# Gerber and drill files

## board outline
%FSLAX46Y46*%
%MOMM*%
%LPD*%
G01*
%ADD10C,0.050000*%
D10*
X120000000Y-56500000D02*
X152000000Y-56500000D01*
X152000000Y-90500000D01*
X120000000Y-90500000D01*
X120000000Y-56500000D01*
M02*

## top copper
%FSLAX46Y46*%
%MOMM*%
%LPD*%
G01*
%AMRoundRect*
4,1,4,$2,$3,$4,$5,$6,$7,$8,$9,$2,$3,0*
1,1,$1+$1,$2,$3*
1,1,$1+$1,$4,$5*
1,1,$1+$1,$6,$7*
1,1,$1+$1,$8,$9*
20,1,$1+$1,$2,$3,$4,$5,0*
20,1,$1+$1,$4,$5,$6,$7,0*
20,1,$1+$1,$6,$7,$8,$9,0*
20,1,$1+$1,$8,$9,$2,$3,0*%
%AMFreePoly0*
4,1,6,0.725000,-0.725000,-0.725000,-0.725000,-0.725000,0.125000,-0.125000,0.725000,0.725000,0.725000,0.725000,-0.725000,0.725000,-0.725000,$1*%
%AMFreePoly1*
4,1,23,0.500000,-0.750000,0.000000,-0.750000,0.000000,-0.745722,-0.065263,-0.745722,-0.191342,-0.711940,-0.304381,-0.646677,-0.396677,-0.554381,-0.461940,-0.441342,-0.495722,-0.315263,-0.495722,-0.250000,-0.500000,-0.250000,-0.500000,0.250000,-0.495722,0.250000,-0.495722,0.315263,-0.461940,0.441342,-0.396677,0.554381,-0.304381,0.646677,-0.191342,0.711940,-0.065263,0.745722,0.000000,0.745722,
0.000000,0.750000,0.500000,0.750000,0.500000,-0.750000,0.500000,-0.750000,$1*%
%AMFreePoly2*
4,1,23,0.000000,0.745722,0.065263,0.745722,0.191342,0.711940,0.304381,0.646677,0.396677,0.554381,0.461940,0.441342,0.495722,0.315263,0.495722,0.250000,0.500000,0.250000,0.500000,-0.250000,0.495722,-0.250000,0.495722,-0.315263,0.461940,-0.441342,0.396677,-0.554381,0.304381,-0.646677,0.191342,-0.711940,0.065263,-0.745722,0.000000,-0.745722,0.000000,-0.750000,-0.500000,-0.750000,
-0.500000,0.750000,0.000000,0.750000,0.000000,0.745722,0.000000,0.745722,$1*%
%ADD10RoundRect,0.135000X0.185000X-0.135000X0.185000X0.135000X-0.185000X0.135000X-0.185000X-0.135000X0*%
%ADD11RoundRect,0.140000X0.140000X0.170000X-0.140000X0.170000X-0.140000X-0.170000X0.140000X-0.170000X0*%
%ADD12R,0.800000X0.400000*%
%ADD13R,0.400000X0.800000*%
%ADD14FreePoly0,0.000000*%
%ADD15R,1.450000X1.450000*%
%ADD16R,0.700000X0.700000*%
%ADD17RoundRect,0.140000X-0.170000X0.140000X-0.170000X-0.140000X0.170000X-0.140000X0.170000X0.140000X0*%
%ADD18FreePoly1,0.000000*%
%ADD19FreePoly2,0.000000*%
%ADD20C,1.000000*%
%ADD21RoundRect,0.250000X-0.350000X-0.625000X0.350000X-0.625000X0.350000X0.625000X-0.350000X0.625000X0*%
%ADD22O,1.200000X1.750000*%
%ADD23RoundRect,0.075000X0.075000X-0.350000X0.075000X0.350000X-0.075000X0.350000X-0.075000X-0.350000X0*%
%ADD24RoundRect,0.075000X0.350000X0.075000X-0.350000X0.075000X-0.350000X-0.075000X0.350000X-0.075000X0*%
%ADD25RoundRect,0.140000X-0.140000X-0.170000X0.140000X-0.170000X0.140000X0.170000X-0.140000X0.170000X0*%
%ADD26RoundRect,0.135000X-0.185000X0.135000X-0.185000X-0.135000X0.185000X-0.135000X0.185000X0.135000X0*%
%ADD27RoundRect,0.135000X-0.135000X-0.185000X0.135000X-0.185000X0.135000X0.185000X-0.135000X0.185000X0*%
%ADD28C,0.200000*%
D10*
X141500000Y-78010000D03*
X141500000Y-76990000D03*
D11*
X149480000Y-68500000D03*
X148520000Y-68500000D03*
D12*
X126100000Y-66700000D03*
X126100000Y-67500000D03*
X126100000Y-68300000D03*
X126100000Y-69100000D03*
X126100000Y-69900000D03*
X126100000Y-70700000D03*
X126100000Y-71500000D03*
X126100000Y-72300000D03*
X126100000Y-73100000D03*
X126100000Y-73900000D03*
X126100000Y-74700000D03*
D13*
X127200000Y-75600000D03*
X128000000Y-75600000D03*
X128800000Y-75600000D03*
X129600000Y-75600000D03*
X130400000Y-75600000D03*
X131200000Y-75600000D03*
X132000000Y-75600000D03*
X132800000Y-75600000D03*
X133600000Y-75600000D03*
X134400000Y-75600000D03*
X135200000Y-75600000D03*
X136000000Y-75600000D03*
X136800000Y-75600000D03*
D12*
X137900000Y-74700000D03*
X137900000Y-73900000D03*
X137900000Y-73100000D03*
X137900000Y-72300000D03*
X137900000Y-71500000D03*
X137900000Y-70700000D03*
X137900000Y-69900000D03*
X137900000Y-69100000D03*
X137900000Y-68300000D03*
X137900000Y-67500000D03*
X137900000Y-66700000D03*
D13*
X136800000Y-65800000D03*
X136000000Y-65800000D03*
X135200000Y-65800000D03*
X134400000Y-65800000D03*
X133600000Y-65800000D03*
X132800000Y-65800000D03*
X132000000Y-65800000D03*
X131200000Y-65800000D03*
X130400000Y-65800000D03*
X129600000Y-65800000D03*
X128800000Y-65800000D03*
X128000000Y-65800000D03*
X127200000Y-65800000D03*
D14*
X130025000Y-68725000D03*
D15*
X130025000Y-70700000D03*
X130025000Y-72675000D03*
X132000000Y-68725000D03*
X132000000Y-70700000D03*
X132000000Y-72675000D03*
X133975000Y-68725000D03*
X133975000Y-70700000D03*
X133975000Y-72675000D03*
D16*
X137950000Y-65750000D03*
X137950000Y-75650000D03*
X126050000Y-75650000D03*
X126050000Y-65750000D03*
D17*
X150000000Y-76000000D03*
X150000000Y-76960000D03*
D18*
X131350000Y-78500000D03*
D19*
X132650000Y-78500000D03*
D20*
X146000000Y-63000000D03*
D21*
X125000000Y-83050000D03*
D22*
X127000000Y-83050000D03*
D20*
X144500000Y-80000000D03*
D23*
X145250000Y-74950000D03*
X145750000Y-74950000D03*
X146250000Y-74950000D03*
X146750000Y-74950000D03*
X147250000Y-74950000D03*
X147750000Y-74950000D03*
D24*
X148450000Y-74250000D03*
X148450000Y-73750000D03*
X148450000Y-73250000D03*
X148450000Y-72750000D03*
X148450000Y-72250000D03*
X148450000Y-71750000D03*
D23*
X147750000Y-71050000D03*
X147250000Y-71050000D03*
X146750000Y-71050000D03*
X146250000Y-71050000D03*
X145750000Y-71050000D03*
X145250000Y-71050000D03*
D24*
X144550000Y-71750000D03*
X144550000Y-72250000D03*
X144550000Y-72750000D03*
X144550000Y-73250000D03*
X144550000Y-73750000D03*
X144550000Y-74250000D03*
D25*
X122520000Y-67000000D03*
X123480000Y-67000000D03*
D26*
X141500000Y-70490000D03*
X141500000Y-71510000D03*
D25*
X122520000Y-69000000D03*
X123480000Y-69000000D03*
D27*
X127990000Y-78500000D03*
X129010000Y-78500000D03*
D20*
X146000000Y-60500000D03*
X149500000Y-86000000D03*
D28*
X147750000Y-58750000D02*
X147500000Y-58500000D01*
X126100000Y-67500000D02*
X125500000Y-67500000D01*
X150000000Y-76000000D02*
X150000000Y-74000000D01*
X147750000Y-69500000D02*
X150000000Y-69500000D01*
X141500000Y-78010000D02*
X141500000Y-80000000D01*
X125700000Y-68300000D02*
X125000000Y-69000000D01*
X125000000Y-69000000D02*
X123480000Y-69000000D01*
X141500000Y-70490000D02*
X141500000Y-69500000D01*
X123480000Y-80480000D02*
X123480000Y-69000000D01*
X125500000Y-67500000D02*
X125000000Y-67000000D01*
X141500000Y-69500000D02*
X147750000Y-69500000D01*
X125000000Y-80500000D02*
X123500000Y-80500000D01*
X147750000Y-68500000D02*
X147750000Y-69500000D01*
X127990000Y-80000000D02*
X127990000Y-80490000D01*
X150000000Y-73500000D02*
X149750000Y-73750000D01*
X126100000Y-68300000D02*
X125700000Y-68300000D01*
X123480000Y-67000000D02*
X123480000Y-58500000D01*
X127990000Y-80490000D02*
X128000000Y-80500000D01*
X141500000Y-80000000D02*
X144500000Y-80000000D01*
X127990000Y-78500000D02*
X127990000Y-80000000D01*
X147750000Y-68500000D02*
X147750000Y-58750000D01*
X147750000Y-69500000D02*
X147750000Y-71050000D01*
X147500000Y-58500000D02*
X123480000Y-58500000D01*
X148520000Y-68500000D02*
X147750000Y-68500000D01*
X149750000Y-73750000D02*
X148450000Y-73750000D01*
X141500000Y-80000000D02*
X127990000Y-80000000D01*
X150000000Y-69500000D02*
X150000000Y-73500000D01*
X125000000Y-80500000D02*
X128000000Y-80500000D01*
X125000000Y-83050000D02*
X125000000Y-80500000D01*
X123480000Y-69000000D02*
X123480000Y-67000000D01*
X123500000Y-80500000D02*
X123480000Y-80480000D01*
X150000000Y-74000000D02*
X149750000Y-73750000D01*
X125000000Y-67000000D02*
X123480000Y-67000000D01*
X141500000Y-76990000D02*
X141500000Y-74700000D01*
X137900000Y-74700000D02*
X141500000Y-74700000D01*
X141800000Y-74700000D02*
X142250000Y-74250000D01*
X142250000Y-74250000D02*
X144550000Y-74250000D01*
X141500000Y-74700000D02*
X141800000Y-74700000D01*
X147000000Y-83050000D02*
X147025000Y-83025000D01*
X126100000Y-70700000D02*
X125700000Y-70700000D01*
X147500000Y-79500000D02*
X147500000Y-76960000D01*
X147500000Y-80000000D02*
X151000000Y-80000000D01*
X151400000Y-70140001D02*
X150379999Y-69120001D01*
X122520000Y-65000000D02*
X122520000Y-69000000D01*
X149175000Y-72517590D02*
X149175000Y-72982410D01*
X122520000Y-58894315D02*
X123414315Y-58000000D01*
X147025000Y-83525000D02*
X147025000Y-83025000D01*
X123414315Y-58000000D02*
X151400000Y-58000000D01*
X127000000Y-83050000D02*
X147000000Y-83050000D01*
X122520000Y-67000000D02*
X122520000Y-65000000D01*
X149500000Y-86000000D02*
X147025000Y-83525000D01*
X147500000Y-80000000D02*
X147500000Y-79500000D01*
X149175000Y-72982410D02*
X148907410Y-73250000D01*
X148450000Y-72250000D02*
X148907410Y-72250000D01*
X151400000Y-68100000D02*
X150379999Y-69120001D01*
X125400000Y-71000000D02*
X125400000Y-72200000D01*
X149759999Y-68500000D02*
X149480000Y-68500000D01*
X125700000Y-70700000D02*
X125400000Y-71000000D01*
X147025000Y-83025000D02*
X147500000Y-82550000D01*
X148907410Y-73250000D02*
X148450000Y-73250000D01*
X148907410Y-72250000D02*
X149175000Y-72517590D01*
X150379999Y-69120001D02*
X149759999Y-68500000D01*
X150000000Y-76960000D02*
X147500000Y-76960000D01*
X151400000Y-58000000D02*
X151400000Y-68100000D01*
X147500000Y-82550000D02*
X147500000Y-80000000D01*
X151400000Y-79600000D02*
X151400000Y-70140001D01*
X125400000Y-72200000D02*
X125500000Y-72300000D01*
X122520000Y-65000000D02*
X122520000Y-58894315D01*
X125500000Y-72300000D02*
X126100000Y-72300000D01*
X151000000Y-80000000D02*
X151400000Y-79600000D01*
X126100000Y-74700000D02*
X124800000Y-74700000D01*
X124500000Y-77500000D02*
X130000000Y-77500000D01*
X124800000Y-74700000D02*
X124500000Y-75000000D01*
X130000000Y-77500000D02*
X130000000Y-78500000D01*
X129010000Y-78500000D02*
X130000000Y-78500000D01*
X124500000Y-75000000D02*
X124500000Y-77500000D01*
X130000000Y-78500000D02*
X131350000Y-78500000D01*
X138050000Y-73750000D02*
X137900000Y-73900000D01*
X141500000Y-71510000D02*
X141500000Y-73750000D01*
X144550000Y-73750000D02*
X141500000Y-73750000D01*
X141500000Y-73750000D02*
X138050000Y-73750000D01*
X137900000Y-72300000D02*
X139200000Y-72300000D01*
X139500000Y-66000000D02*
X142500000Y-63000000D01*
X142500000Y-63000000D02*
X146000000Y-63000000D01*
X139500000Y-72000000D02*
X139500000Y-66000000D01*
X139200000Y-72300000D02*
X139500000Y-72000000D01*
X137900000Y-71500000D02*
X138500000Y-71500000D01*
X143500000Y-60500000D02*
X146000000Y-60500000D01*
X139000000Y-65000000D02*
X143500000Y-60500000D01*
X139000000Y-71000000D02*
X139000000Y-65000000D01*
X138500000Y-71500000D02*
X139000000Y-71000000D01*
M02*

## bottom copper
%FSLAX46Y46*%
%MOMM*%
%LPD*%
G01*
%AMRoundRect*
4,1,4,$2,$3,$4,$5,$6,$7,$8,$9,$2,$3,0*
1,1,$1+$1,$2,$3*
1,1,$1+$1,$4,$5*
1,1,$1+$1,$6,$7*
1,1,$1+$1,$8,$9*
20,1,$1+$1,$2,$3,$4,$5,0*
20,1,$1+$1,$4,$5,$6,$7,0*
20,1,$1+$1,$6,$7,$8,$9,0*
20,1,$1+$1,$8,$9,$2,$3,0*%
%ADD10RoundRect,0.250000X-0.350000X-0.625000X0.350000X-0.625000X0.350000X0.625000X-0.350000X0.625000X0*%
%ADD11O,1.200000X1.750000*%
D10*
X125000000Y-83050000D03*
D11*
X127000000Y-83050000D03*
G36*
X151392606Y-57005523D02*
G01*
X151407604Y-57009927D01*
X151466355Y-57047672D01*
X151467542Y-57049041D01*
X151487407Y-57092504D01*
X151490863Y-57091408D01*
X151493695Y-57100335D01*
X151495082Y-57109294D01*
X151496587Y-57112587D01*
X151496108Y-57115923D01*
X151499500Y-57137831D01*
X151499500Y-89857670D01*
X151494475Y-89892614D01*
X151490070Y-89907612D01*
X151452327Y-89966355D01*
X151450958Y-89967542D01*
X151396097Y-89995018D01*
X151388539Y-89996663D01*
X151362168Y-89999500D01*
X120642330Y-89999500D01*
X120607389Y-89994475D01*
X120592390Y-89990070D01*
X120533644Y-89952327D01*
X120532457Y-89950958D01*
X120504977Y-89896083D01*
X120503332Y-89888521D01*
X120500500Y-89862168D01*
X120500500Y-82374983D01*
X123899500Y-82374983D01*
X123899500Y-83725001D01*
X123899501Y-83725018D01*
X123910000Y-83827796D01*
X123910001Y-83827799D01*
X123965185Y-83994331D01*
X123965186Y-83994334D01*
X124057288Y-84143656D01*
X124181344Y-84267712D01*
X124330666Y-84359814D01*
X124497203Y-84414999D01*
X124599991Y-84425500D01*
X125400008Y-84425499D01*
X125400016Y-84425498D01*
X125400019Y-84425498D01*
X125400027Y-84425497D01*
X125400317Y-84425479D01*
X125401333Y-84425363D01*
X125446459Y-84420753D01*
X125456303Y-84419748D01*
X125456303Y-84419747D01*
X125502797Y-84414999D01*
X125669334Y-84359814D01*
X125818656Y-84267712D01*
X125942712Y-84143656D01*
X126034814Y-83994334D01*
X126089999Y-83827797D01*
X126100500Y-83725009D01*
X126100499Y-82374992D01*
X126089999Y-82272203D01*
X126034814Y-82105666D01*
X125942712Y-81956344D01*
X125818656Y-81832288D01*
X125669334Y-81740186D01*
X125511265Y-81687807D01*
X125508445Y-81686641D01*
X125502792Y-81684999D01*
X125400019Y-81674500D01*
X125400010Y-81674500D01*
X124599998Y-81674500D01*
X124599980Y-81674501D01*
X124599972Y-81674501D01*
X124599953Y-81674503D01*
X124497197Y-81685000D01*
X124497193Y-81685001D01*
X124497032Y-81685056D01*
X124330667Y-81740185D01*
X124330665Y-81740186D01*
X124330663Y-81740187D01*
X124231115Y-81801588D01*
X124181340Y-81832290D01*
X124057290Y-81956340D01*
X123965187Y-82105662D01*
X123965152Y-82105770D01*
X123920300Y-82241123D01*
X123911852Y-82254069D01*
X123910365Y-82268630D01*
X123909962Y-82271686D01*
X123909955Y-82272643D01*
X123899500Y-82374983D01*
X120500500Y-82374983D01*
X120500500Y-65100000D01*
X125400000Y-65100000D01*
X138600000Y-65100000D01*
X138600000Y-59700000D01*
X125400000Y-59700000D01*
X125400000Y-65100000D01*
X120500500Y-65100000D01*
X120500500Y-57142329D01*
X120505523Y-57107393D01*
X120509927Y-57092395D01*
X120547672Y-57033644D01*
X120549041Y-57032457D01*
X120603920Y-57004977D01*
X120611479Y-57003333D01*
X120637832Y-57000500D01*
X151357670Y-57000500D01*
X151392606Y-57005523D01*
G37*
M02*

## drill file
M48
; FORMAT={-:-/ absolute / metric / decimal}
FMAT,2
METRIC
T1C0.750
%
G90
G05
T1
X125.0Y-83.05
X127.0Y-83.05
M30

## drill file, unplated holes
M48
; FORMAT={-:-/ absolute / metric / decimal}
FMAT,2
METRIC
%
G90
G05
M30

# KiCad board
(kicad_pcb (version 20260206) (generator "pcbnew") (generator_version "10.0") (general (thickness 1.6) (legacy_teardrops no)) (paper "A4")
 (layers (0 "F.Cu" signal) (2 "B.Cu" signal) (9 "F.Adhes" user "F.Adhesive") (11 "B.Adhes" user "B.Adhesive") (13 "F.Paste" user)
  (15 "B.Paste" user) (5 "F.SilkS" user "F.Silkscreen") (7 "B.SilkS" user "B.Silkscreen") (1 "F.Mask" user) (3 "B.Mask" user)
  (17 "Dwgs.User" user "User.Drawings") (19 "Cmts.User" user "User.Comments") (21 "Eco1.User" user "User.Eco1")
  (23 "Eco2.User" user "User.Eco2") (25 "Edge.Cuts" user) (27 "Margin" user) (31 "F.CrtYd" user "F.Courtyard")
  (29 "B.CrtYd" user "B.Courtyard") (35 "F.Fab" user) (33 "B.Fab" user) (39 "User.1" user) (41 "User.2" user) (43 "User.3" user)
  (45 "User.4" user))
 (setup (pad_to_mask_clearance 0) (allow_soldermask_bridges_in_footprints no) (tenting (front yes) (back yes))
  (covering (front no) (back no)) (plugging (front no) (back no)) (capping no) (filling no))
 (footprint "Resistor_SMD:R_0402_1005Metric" (layer "F.Cu") (at 141.5 77.5 90)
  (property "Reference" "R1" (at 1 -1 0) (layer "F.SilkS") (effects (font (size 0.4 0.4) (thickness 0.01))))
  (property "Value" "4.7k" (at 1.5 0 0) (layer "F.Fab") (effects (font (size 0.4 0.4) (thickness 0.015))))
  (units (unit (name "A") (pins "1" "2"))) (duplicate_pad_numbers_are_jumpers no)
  (pad "1" smd roundrect (at -0.51 0 90) (size 0.54 0.64) (layers "F.Cu" "F.Mask" "F.Paste") (roundrect_rratio 0.25) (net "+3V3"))
  (pad "2" smd roundrect (at 0.51 0 90) (size 0.54 0.64) (layers "F.Cu" "F.Mask" "F.Paste") (roundrect_rratio 0.25) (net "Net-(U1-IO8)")))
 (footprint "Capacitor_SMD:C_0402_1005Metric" (layer "F.Cu") (at 149 68.5 180)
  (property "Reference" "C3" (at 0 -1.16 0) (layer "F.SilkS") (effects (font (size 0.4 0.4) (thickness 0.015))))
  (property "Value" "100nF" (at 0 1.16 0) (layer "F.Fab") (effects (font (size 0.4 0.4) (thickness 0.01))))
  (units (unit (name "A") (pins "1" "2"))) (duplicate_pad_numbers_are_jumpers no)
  (pad "1" smd roundrect (at -0.48 0 180) (size 0.56 0.62) (layers "F.Cu" "F.Mask" "F.Paste") (roundrect_rratio 0.25) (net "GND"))
  (pad "2" smd roundrect (at 0.48 0 180) (size 0.56 0.62) (layers "F.Cu" "F.Mask" "F.Paste") (roundrect_rratio 0.25) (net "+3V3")))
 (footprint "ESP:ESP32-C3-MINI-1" (layer "F.Cu") (at 132 68)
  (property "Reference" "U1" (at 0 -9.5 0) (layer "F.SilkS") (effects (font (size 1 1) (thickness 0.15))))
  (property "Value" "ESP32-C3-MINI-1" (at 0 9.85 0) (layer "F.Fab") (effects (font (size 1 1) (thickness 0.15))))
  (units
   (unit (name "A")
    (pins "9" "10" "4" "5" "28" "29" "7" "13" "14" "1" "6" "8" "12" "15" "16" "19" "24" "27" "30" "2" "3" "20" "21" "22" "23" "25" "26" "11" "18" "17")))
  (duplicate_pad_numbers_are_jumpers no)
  (pad "1" smd rect (at -5.9 -1.3 90) (size 0.4 0.8) (layers "F.Cu" "F.Mask" "F.Paste") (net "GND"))
  (pad "2" smd rect (at -5.9 -0.5 90) (size 0.4 0.8) (layers "F.Cu" "F.Mask" "F.Paste") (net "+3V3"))
  (pad "3" smd rect (at -5.9 0.3 90) (size 0.4 0.8) (layers "F.Cu" "F.Mask" "F.Paste") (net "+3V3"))
  (pad "4" smd rect (at -5.9 1.1 90) (size 0.4 0.8) (layers "F.Cu" "F.Mask" "F.Paste") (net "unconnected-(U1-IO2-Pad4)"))
  (pad "5" smd rect (at -5.9 1.9 90) (size 0.4 0.8) (layers "F.Cu" "F.Mask" "F.Paste") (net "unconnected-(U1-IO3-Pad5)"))
  (pad "6" smd rect (at -5.9 2.7 90) (size 0.4 0.8) (layers "F.Cu" "F.Mask" "F.Paste") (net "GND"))
  (pad "7" smd rect (at -5.9 3.5 90) (size 0.4 0.8) (layers "F.Cu" "F.Mask" "F.Paste") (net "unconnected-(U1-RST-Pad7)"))
  (pad "8" smd rect (at -5.9 4.3 90) (size 0.4 0.8) (layers "F.Cu" "F.Mask" "F.Paste") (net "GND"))
  (pad "9" smd rect (at -5.9 5.1 90) (size 0.4 0.8) (layers "F.Cu" "F.Mask" "F.Paste") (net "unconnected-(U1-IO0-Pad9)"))
  (pad "10" smd rect (at -5.9 5.9 90) (size 0.4 0.8) (layers "F.Cu" "F.Mask" "F.Paste") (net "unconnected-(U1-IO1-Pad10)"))
  (pad "11" smd rect (at -5.9 6.7 90) (size 0.4 0.8) (layers "F.Cu" "F.Mask" "F.Paste") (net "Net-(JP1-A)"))
  (pad "12" smd rect (at -4.8 7.6) (size 0.4 0.8) (layers "F.Cu" "F.Mask" "F.Paste") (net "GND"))
  (pad "13" smd rect (at -4 7.6) (size 0.4 0.8) (layers "F.Cu" "F.Mask" "F.Paste") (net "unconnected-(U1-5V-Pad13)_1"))
  (pad "14" smd rect (at -3.2 7.6) (size 0.4 0.8) (layers "F.Cu" "F.Mask" "F.Paste") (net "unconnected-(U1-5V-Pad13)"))
  (pad "15" smd rect (at -2.4 7.6) (size 0.4 0.8) (layers "F.Cu" "F.Mask" "F.Paste") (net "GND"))
  (pad "16" smd rect (at -1.6 7.6) (size 0.4 0.8) (layers "F.Cu" "F.Mask" "F.Paste") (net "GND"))
  (pad "17" smd rect (at -0.8 7.6) (size 0.4 0.8) (layers "F.Cu" "F.Mask" "F.Paste") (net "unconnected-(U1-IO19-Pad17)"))
  (pad "18" smd rect (at 0 7.6) (size 0.4 0.8) (layers "F.Cu" "F.Mask" "F.Paste") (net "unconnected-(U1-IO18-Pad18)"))
  (pad "19" smd rect (at 0.8 7.6) (size 0.4 0.8) (layers "F.Cu" "F.Mask" "F.Paste") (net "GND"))
  (pad "20" smd rect (at 1.6 7.6) (size 0.4 0.8) (layers "F.Cu" "F.Mask" "F.Paste") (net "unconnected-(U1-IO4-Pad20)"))
  (pad "21" smd rect (at 2.4 7.6) (size 0.4 0.8) (layers "F.Cu" "F.Mask" "F.Paste") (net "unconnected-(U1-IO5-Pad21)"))
  (pad "22" smd rect (at 3.2 7.6) (size 0.4 0.8) (layers "F.Cu" "F.Mask" "F.Paste") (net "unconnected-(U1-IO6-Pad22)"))
  (pad "23" smd rect (at 4 7.6) (size 0.4 0.8) (layers "F.Cu" "F.Mask" "F.Paste") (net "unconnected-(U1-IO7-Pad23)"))
  (pad "24" smd rect (at 4.8 7.6) (size 0.4 0.8) (layers "F.Cu" "F.Mask" "F.Paste") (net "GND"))
  (pad "25" smd rect (at 5.9 6.7 90) (size 0.4 0.8) (layers "F.Cu" "F.Mask" "F.Paste") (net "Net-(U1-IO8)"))
  (pad "26" smd rect (at 5.9 5.9 90) (size 0.4 0.8) (layers "F.Cu" "F.Mask" "F.Paste") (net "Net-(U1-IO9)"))
  (pad "27" smd rect (at 5.9 5.1 90) (size 0.4 0.8) (layers "F.Cu" "F.Mask" "F.Paste") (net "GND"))
  (pad "28" smd rect (at 5.9 4.3 90) (size 0.4 0.8) (layers "F.Cu" "F.Mask" "F.Paste") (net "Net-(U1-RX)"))
  (pad "29" smd rect (at 5.9 3.5 90) (size 0.4 0.8) (layers "F.Cu" "F.Mask" "F.Paste") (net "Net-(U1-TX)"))
  (pad "30" smd rect (at 5.9 2.7 90) (size 0.4 0.8) (layers "F.Cu" "F.Mask" "F.Paste") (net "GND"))
  (pad "31" smd rect (at 5.9 1.9 90) (size 0.4 0.8) (layers "F.Cu" "F.Mask" "F.Paste"))
  (pad "32" smd rect (at 5.9 1.1 90) (size 0.4 0.8) (layers "F.Cu" "F.Mask" "F.Paste"))
  (pad "33" smd rect (at 5.9 0.3 90) (size 0.4 0.8) (layers "F.Cu" "F.Mask" "F.Paste"))
  (pad "34" smd rect (at 5.9 -0.5 90) (size 0.4 0.8) (layers "F.Cu" "F.Mask" "F.Paste"))
  (pad "35" smd rect (at 5.9 -1.3 90) (size 0.4 0.8) (layers "F.Cu" "F.Mask" "F.Paste"))
  (pad "36" smd rect (at 4.8 -2.2) (size 0.4 0.8) (layers "F.Cu" "F.Mask" "F.Paste"))
  (pad "37" smd rect (at 4 -2.2) (size 0.4 0.8) (layers "F.Cu" "F.Mask" "F.Paste"))
  (pad "38" smd rect (at 3.2 -2.2) (size 0.4 0.8) (layers "F.Cu" "F.Mask" "F.Paste"))
  (pad "39" smd rect (at 2.4 -2.2) (size 0.4 0.8) (layers "F.Cu" "F.Mask" "F.Paste"))
  (pad "40" smd rect (at 1.6 -2.2) (size 0.4 0.8) (layers "F.Cu" "F.Mask" "F.Paste"))
  (pad "41" smd rect (at 0.8 -2.2) (size 0.4 0.8) (layers "F.Cu" "F.Mask" "F.Paste"))
  (pad "42" smd rect (at 0 -2.2) (size 0.4 0.8) (layers "F.Cu" "F.Mask" "F.Paste"))
  (pad "43" smd rect (at -0.8 -2.2) (size 0.4 0.8) (layers "F.Cu" "F.Mask" "F.Paste"))
  (pad "44" smd rect (at -1.6 -2.2) (size 0.4 0.8) (layers "F.Cu" "F.Mask" "F.Paste"))
  (pad "45" smd rect (at -2.4 -2.2) (size 0.4 0.8) (layers "F.Cu" "F.Mask" "F.Paste"))
  (pad "46" smd rect (at -3.2 -2.2) (size 0.4 0.8) (layers "F.Cu" "F.Mask" "F.Paste"))
  (pad "47" smd rect (at -4 -2.2) (size 0.4 0.8) (layers "F.Cu" "F.Mask" "F.Paste"))
  (pad "48" smd rect (at -4.8 -2.2) (size 0.4 0.8) (layers "F.Cu" "F.Mask" "F.Paste"))
  (pad "49" smd custom (at -1.975 0.725) (size 0.8 0.8) (layers "F.Cu" "F.Mask" "F.Paste") (zone_connect 2) (thermal_bridge_angle 45)
   (options (clearance outline) (anchor rect)) (primitives))
  (pad "49" smd rect (at -1.975 2.7 90) (size 1.45 1.45) (layers "F.Cu" "F.Mask" "F.Paste") (zone_connect 2))
  (pad "49" smd rect (at -1.975 4.675 90) (size 1.45 1.45) (layers "F.Cu" "F.Mask" "F.Paste") (zone_connect 2))
  (pad "49" smd rect (at 0 0.725 90) (size 1.45 1.45) (layers "F.Cu" "F.Mask" "F.Paste") (zone_connect 2))
  (pad "49" smd rect (at 0 2.7 90) (size 1.45 1.45) (layers "F.Cu" "F.Mask" "F.Paste") (zone_connect 2))
  (pad "49" smd rect (at 0 4.675 90) (size 1.45 1.45) (layers "F.Cu" "F.Mask" "F.Paste") (zone_connect 2))
  (pad "49" smd rect (at 1.975 0.725 90) (size 1.45 1.45) (layers "F.Cu" "F.Mask" "F.Paste") (zone_connect 2))
  (pad "49" smd rect (at 1.975 2.7 90) (size 1.45 1.45) (layers "F.Cu" "F.Mask" "F.Paste") (zone_connect 2))
  (pad "49" smd rect (at 1.975 4.675 90) (size 1.45 1.45) (layers "F.Cu" "F.Mask" "F.Paste") (zone_connect 2))
  (pad "50" smd rect (at 5.95 -2.25 90) (size 0.7 0.7) (layers "F.Cu" "F.Mask" "F.Paste"))
  (pad "51" smd rect (at 5.95 7.65 90) (size 0.7 0.7) (layers "F.Cu" "F.Mask" "F.Paste"))
  (pad "52" smd rect (at -5.95 7.65 90) (size 0.7 0.7) (layers "F.Cu" "F.Mask" "F.Paste"))
  (pad "53" smd rect (at -5.95 -2.25 90) (size 0.7 0.7) (layers "F.Cu" "F.Mask" "F.Paste"))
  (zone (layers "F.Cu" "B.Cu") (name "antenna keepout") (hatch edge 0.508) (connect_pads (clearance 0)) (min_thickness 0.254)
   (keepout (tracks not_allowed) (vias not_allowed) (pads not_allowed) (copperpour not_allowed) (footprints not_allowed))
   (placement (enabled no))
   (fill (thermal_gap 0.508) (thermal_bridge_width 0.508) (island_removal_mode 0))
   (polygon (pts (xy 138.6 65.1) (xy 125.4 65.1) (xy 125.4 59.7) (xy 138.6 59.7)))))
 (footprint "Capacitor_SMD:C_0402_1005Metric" (layer "F.Cu") (at 150 76.48 -90)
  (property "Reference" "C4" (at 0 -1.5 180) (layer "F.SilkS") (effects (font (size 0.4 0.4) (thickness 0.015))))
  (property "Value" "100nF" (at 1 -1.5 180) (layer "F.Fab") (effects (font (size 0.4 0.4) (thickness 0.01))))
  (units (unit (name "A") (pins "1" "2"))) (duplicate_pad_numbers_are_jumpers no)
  (pad "1" smd roundrect (at -0.48 0 270) (size 0.56 0.62) (layers "F.Cu" "F.Mask" "F.Paste") (roundrect_rratio 0.25) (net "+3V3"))
  (pad "2" smd roundrect (at 0.48 0 270) (size 0.56 0.62) (layers "F.Cu" "F.Mask" "F.Paste") (roundrect_rratio 0.25) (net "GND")))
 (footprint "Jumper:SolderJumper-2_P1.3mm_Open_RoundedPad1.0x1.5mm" (layer "F.Cu") (at 132 78.5)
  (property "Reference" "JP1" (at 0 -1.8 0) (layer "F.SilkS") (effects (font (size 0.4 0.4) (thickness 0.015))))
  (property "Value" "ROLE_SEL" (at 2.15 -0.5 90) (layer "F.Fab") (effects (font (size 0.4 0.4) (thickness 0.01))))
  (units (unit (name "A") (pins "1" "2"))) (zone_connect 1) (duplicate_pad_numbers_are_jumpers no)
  (pad "1" smd custom (at -0.65 0) (size 1 0.5) (layers "F.Cu" "F.Mask") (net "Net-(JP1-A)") (zone_connect 2) (thermal_bridge_angle 45)
   (options (clearance outline) (anchor rect)) (primitives))
  (pad "2" smd custom (at 0.65 0) (size 1 0.5) (layers "F.Cu" "F.Mask") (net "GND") (zone_connect 2) (thermal_bridge_angle 45)
   (options (clearance outline) (anchor rect)) (primitives)))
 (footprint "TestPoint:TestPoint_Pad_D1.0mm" (layer "F.Cu") (at 146 63)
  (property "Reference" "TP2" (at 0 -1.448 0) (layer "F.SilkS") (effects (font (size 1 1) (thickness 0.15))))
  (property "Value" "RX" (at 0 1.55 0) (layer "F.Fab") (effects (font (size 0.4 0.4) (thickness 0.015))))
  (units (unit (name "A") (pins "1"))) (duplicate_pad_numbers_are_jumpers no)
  (pad "1" smd circle (at 0 0) (size 1 1) (layers "F.Cu" "F.Mask") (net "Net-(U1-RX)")))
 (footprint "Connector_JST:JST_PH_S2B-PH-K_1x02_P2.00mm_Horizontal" (layer "F.Cu") (at 125 83.05)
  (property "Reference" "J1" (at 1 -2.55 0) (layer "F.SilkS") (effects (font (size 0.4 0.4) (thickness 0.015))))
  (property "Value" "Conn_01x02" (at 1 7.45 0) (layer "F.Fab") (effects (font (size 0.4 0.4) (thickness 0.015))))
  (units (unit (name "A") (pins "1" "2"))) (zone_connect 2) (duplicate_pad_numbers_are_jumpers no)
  (pad "1" thru_hole roundrect (at 0 0) (size 1.2 1.75) (drill 0.75) (layers "*.Cu" "*.Mask") (remove_unused_layers no)
   (roundrect_rratio 0.208333) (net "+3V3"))
  (pad "2" thru_hole oval (at 2 0) (size 1.2 1.75) (drill 0.75) (layers "*.Cu" "*.Mask") (remove_unused_layers no) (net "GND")))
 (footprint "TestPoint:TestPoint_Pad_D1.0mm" (layer "F.Cu") (at 144.5 80 180)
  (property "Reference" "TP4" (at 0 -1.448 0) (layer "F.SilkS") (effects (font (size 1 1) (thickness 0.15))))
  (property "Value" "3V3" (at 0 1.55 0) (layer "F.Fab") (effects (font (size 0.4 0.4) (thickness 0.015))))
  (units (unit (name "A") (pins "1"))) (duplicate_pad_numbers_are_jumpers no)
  (pad "1" smd circle (at 0 0 180) (size 1 1) (layers "F.Cu" "F.Mask") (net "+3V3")))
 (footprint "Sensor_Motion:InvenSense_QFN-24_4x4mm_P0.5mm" (layer "F.Cu") (at 146.5 73 90)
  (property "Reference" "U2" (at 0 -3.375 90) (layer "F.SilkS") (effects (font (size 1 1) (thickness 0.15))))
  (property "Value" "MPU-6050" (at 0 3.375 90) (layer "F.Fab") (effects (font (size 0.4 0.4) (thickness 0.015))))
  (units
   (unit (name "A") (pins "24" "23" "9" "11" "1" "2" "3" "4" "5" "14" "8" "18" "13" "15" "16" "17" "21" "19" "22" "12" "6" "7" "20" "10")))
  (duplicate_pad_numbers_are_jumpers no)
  (pad "1" smd roundrect (at -1.95 -1.25 90) (size 0.85 0.3) (layers "F.Cu" "F.Mask" "F.Paste") (roundrect_rratio 0.25)
   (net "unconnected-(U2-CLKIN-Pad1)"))
  (pad "2" smd roundrect (at -1.95 -0.75 90) (size 0.85 0.3) (layers "F.Cu" "F.Mask" "F.Paste") (roundrect_rratio 0.25)
   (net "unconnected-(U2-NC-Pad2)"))
  (pad "3" smd roundrect (at -1.95 -0.25 90) (size 0.85 0.3) (layers "F.Cu" "F.Mask" "F.Paste") (roundrect_rratio 0.25)
   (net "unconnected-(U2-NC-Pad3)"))
  (pad "4" smd roundrect (at -1.95 0.25 90) (size 0.85 0.3) (layers "F.Cu" "F.Mask" "F.Paste") (roundrect_rratio 0.25)
   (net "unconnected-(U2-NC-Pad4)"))
  (pad "5" smd roundrect (at -1.95 0.75 90) (size 0.85 0.3) (layers "F.Cu" "F.Mask" "F.Paste") (roundrect_rratio 0.25)
   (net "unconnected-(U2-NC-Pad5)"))
  (pad "6" smd roundrect (at -1.95 1.25 90) (size 0.85 0.3) (layers "F.Cu" "F.Mask" "F.Paste") (roundrect_rratio 0.25)
   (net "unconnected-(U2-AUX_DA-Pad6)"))
  (pad "7" smd roundrect (at -1.25 1.95 180) (size 0.85 0.3) (layers "F.Cu" "F.Mask" "F.Paste") (roundrect_rratio 0.25)
   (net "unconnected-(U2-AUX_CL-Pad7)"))
  (pad "8" smd roundrect (at -0.75 1.95 180) (size 0.85 0.3) (layers "F.Cu" "F.Mask" "F.Paste") (roundrect_rratio 0.25) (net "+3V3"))
  (pad "9" smd roundrect (at -0.25 1.95 180) (size 0.85 0.3) (layers "F.Cu" "F.Mask" "F.Paste") (roundrect_rratio 0.25) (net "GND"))
  (pad "10" smd roundrect (at 0.25 1.95 180) (size 0.85 0.3) (layers "F.Cu" "F.Mask" "F.Paste") (roundrect_rratio 0.25)
   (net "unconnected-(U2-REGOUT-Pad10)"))
  (pad "11" smd roundrect (at 0.75 1.95 180) (size 0.85 0.3) (layers "F.Cu" "F.Mask" "F.Paste") (roundrect_rratio 0.25) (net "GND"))
  (pad "12" smd roundrect (at 1.25 1.95 180) (size 0.85 0.3) (layers "F.Cu" "F.Mask" "F.Paste") (roundrect_rratio 0.25)
   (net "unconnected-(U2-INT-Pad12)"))
  (pad "13" smd roundrect (at 1.95 1.25 90) (size 0.85 0.3) (layers "F.Cu" "F.Mask" "F.Paste") (roundrect_rratio 0.25) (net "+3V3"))
  (pad "14" smd roundrect (at 1.95 0.75 90) (size 0.85 0.3) (layers "F.Cu" "F.Mask" "F.Paste") (roundrect_rratio 0.25)
   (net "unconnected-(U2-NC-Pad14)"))
  (pad "15" smd roundrect (at 1.95 0.25 90) (size 0.85 0.3) (layers "F.Cu" "F.Mask" "F.Paste") (roundrect_rratio 0.25)
   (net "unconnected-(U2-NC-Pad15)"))
  (pad "16" smd roundrect (at 1.95 -0.25 90) (size 0.85 0.3) (layers "F.Cu" "F.Mask" "F.Paste") (roundrect_rratio 0.25)
   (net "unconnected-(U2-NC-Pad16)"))
  (pad "17" smd roundrect (at 1.95 -0.75 90) (size 0.85 0.3) (layers "F.Cu" "F.Mask" "F.Paste") (roundrect_rratio 0.25)
   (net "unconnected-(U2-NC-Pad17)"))
  (pad "18" smd roundrect (at 1.95 -1.25 90) (size 0.85 0.3) (layers "F.Cu" "F.Mask" "F.Paste") (roundrect_rratio 0.25) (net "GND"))
  (pad "19" smd roundrect (at 1.25 -1.95 180) (size 0.85 0.3) (layers "F.Cu" "F.Mask" "F.Paste") (roundrect_rratio 0.25)
   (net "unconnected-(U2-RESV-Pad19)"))
  (pad "20" smd roundrect (at 0.75 -1.95 180) (size 0.85 0.3) (layers "F.Cu" "F.Mask" "F.Paste") (roundrect_rratio 0.25)
   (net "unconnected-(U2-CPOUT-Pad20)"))
  (pad "21" smd roundrect (at 0.25 -1.95 180) (size 0.85 0.3) (layers "F.Cu" "F.Mask" "F.Paste") (roundrect_rratio 0.25)
   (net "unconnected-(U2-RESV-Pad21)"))
  (pad "22" smd roundrect (at -0.25 -1.95 180) (size 0.85 0.3) (layers "F.Cu" "F.Mask" "F.Paste") (roundrect_rratio 0.25)
   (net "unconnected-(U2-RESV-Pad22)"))
  (pad "23" smd roundrect (at -0.75 -1.95 180) (size 0.85 0.3) (layers "F.Cu" "F.Mask" "F.Paste") (roundrect_rratio 0.25)
   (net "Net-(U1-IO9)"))
  (pad "24" smd roundrect (at -1.25 -1.95 180) (size 0.85 0.3) (layers "F.Cu" "F.Mask" "F.Paste") (roundrect_rratio 0.25)
   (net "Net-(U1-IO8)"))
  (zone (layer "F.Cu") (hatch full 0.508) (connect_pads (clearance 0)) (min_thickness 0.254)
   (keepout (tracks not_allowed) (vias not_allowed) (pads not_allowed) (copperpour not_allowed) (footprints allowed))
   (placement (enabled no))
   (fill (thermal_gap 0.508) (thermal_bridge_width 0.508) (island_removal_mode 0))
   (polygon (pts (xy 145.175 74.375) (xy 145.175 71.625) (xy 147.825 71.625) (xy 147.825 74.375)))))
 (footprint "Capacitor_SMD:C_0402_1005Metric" (layer "F.Cu") (at 123 67)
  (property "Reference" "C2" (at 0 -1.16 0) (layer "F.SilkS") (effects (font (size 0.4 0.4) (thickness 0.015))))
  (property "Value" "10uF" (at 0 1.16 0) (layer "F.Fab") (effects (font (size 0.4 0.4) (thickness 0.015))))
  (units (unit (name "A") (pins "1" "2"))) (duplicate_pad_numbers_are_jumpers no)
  (pad "1" smd roundrect (at -0.48 0) (size 0.56 0.62) (layers "F.Cu" "F.Mask" "F.Paste") (roundrect_rratio 0.25) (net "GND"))
  (pad "2" smd roundrect (at 0.48 0) (size 0.56 0.62) (layers "F.Cu" "F.Mask" "F.Paste") (roundrect_rratio 0.25) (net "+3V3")))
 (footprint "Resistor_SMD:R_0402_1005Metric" (layer "F.Cu") (at 141.5 71 -90)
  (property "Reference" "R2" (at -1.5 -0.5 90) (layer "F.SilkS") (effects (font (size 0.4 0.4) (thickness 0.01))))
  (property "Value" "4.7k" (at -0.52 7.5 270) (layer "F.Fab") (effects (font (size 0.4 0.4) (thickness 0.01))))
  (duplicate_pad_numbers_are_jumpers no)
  (pad "1" smd roundrect (at -0.51 0 270) (size 0.54 0.64) (layers "F.Cu" "F.Mask" "F.Paste") (roundrect_rratio 0.25) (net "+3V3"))
  (pad "2" smd roundrect (at 0.51 0 270) (size 0.54 0.64) (layers "F.Cu" "F.Mask" "F.Paste") (roundrect_rratio 0.25) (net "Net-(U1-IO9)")))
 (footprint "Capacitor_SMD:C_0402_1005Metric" (layer "F.Cu") (at 123 69)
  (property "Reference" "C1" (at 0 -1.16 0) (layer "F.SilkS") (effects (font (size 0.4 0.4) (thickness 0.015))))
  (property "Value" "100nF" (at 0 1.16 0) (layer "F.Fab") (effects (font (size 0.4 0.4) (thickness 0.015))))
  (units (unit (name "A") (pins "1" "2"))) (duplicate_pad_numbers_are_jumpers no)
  (pad "1" smd roundrect (at -0.48 0) (size 0.56 0.62) (layers "F.Cu" "F.Mask" "F.Paste") (roundrect_rratio 0.25) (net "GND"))
  (pad "2" smd roundrect (at 0.48 0) (size 0.56 0.62) (layers "F.Cu" "F.Mask" "F.Paste") (roundrect_rratio 0.25) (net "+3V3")))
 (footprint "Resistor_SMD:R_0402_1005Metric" (layer "F.Cu") (at 128.5 78.5)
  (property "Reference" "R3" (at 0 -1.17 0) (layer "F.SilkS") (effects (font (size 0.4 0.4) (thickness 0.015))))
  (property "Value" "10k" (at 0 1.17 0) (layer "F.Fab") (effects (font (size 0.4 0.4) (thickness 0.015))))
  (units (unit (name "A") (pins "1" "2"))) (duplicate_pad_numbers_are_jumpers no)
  (pad "1" smd roundrect (at -0.51 0) (size 0.54 0.64) (layers "F.Cu" "F.Mask" "F.Paste") (roundrect_rratio 0.25) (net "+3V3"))
  (pad "2" smd roundrect (at 0.51 0) (size 0.54 0.64) (layers "F.Cu" "F.Mask" "F.Paste") (roundrect_rratio 0.25) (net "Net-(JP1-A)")))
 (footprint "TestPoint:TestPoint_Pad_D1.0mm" (layer "F.Cu") (at 146 60.5)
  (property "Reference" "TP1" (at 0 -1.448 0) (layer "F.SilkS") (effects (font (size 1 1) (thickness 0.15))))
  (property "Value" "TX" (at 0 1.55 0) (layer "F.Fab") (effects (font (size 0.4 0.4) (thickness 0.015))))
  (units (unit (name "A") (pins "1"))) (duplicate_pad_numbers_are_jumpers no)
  (pad "1" smd circle (at 0 0) (size 1 1) (layers "F.Cu" "F.Mask") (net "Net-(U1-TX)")))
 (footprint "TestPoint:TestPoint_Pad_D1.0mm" (layer "F.Cu") (at 149.5 86 90)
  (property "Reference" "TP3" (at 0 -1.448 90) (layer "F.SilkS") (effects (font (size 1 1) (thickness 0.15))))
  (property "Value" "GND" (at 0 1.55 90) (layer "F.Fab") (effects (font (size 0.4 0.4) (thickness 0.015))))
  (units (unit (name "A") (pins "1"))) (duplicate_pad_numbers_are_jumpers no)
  (pad "1" smd circle (at 0 0 90) (size 1 1) (layers "F.Cu" "F.Mask") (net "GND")))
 (gr_rect (start 120 56.5) (end 152 90.5) (stroke (width 0.05) (type default)) (fill no) (layer "Edge.Cuts"))
 (segment (start 147.75 58.75) (end 147.5 58.5) (width 0.2) (layer "F.Cu") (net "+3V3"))
 (segment (start 126.1 67.5) (end 125.5 67.5) (width 0.2) (layer "F.Cu") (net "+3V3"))
 (segment (start 150 76) (end 150 74) (width 0.2) (layer "F.Cu") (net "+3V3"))
 (segment (start 147.75 69.5) (end 150 69.5) (width 0.2) (layer "F.Cu") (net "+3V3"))
 (segment (start 141.5 78.01) (end 141.5 80) (width 0.2) (layer "F.Cu") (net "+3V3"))
 (segment (start 125.7 68.3) (end 125 69) (width 0.2) (layer "F.Cu") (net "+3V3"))
 (segment (start 125 69) (end 123.48 69) (width 0.2) (layer "F.Cu") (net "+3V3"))
 (segment (start 141.5 70.49) (end 141.5 69.5) (width 0.2) (layer "F.Cu") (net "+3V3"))
 (segment (start 123.48 80.48) (end 123.48 69) (width 0.2) (layer "F.Cu") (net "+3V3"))
 (segment (start 125.5 67.5) (end 125 67) (width 0.2) (layer "F.Cu") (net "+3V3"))
 (segment (start 141.5 69.5) (end 147.75 69.5) (width 0.2) (layer "F.Cu") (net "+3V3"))
 (segment (start 125 80.5) (end 123.5 80.5) (width 0.2) (layer "F.Cu") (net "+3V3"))
 (segment (start 147.75 68.5) (end 147.75 69.5) (width 0.2) (layer "F.Cu") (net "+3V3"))
 (segment (start 127.99 80) (end 127.99 80.49) (width 0.2) (layer "F.Cu") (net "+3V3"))
 (segment (start 150 73.5) (end 149.75 73.75) (width 0.2) (layer "F.Cu") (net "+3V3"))
 (segment (start 126.1 68.3) (end 125.7 68.3) (width 0.2) (layer "F.Cu") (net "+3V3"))
 (segment (start 123.48 67) (end 123.48 58.5) (width 0.2) (layer "F.Cu") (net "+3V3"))
 (segment (start 127.99 80.49) (end 128 80.5) (width 0.2) (layer "F.Cu") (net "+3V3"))
 (segment (start 141.5 80) (end 144.5 80) (width 0.2) (layer "F.Cu") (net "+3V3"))
 (segment (start 127.99 78.5) (end 127.99 80) (width 0.2) (layer "F.Cu") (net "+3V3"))
 (segment (start 147.75 68.5) (end 147.75 58.75) (width 0.2) (layer "F.Cu") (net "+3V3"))
 (segment (start 147.75 69.5) (end 147.75 71.05) (width 0.2) (layer "F.Cu") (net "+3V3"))
 (segment (start 147.5 58.5) (end 123.48 58.5) (width 0.2) (layer "F.Cu") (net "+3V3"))
 (segment (start 148.52 68.5) (end 147.75 68.5) (width 0.2) (layer "F.Cu") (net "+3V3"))
 (segment (start 149.75 73.75) (end 148.45 73.75) (width 0.2) (layer "F.Cu") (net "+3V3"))
 (segment (start 141.5 80) (end 127.99 80) (width 0.2) (layer "F.Cu") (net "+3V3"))
 (segment (start 150 69.5) (end 150 73.5) (width 0.2) (layer "F.Cu") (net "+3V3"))
 (segment (start 125 80.5) (end 128 80.5) (width 0.2) (layer "F.Cu") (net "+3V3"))
 (segment (start 125 83.05) (end 125 80.5) (width 0.2) (layer "F.Cu") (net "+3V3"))
 (segment (start 123.48 69) (end 123.48 67) (width 0.2) (layer "F.Cu") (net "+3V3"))
 (segment (start 123.5 80.5) (end 123.48 80.48) (width 0.2) (layer "F.Cu") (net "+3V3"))
 (segment (start 150 74) (end 149.75 73.75) (width 0.2) (layer "F.Cu") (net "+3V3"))
 (segment (start 125 67) (end 123.48 67) (width 0.2) (layer "F.Cu") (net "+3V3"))
 (segment (start 141.5 76.99) (end 141.5 74.7) (width 0.2) (layer "F.Cu") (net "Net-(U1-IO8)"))
 (segment (start 137.9 74.7) (end 141.5 74.7) (width 0.2) (layer "F.Cu") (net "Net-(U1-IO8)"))
 (segment (start 141.8 74.7) (end 142.25 74.25) (width 0.2) (layer "F.Cu") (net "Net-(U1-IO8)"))
 (segment (start 142.25 74.25) (end 144.55 74.25) (width 0.2) (layer "F.Cu") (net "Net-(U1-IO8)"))
 (segment (start 141.5 74.7) (end 141.8 74.7) (width 0.2) (layer "F.Cu") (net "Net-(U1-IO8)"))
 (segment (start 147 83.05) (end 147.025 83.025) (width 0.2) (layer "F.Cu") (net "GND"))
 (segment (start 126.1 70.7) (end 125.7 70.7) (width 0.2) (layer "F.Cu") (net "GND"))
 (segment (start 147.5 79.5) (end 147.5 76.96) (width 0.2) (layer "F.Cu") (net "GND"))
 (segment (start 147.5 80) (end 151 80) (width 0.2) (layer "F.Cu") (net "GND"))
 (segment (start 151.4 70.140001) (end 150.379999 69.120001) (width 0.2) (layer "F.Cu") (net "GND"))
 (segment (start 122.52 65) (end 122.52 69) (width 0.2) (layer "F.Cu") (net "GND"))
 (segment (start 149.175 72.51759) (end 149.175 72.98241) (width 0.2) (layer "F.Cu") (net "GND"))
 (segment (start 122.52 58.894315) (end 123.414315 58) (width 0.2) (layer "F.Cu") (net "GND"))
 (segment (start 147.025 83.525) (end 147.025 83.025) (width 0.2) (layer "F.Cu") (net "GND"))
 (segment (start 123.414315 58) (end 151.4 58) (width 0.2) (layer "F.Cu") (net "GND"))
 (segment (start 127 83.05) (end 147 83.05) (width 0.2) (layer "F.Cu") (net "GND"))
 (segment (start 122.52 67) (end 122.52 65) (width 0.2) (layer "F.Cu") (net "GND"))
 (segment (start 149.5 86) (end 147.025 83.525) (width 0.2) (layer "F.Cu") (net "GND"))
 (segment (start 147.5 80) (end 147.5 79.5) (width 0.2) (layer "F.Cu") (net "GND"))
 (segment (start 149.175 72.98241) (end 148.90741 73.25) (width 0.2) (layer "F.Cu") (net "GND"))
 (segment (start 148.45 72.25) (end 148.90741 72.25) (width 0.2) (layer "F.Cu") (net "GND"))
 (segment (start 151.4 68.1) (end 150.379999 69.120001) (width 0.2) (layer "F.Cu") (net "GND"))
 (segment (start 125.4 71) (end 125.4 72.2) (width 0.2) (layer "F.Cu") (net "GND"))
 (segment (start 149.759999 68.5) (end 149.48 68.5) (width 0.2) (layer "F.Cu") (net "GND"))
 (segment (start 125.7 70.7) (end 125.4 71) (width 0.2) (layer "F.Cu") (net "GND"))
 (segment (start 147.025 83.025) (end 147.5 82.55) (width 0.2) (layer "F.Cu") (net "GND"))
 (segment (start 148.90741 73.25) (end 148.45 73.25) (width 0.2) (layer "F.Cu") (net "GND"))
 (segment (start 148.90741 72.25) (end 149.175 72.51759) (width 0.2) (layer "F.Cu") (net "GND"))
 (segment (start 150.379999 69.120001) (end 149.759999 68.5) (width 0.2) (layer "F.Cu") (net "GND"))
 (segment (start 150 76.96) (end 147.5 76.96) (width 0.2) (layer "F.Cu") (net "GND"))
 (segment (start 151.4 58) (end 151.4 68.1) (width 0.2) (layer "F.Cu") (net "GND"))
 (segment (start 147.5 82.55) (end 147.5 80) (width 0.2) (layer "F.Cu") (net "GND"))
 (segment (start 151.4 79.6) (end 151.4 70.140001) (width 0.2) (layer "F.Cu") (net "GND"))
 (segment (start 125.4 72.2) (end 125.5 72.3) (width 0.2) (layer "F.Cu") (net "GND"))
 (segment (start 122.52 65) (end 122.52 58.894315) (width 0.2) (layer "F.Cu") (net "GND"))
 (segment (start 125.5 72.3) (end 126.1 72.3) (width 0.2) (layer "F.Cu") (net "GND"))
 (segment (start 151 80) (end 151.4 79.6) (width 0.2) (layer "F.Cu") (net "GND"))
 (segment (start 126.1 74.7) (end 124.8 74.7) (width 0.2) (layer "F.Cu") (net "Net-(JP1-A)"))
 (segment (start 124.5 77.5) (end 130 77.5) (width 0.2) (layer "F.Cu") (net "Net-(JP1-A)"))
 (segment (start 124.8 74.7) (end 124.5 75) (width 0.2) (layer "F.Cu") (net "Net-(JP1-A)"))
 (segment (start 130 77.5) (end 130 78.5) (width 0.2) (layer "F.Cu") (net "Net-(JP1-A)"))
 (segment (start 129.01 78.5) (end 130 78.5) (width 0.2) (layer "F.Cu") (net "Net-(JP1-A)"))
 (segment (start 124.5 75) (end 124.5 77.5) (width 0.2) (layer "F.Cu") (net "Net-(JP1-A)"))
 (segment (start 130 78.5) (end 131.35 78.5) (width 0.2) (layer "F.Cu") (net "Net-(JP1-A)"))
 (segment (start 138.05 73.75) (end 137.9 73.9) (width 0.2) (layer "F.Cu") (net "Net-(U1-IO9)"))
 (segment (start 141.5 71.51) (end 141.5 73.75) (width 0.2) (layer "F.Cu") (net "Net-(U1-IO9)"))
 (segment (start 144.55 73.75) (end 141.5 73.75) (width 0.2) (layer "F.Cu") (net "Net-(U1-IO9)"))
 (segment (start 141.5 73.75) (end 138.05 73.75) (width 0.2) (layer "F.Cu") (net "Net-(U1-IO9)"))
 (segment (start 137.9 72.3) (end 139.2 72.3) (width 0.2) (layer "F.Cu") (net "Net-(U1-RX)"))
 (segment (start 139.5 66) (end 142.5 63) (width 0.2) (layer "F.Cu") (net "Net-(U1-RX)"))
 (segment (start 142.5 63) (end 146 63) (width 0.2) (layer "F.Cu") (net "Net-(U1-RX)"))
 (segment (start 139.5 72) (end 139.5 66) (width 0.2) (layer "F.Cu") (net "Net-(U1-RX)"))
 (segment (start 139.2 72.3) (end 139.5 72) (width 0.2) (layer "F.Cu") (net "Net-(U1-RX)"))
 (segment (start 137.9 71.5) (end 138.5 71.5) (width 0.2) (layer "F.Cu") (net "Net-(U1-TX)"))
 (segment (start 143.5 60.5) (end 146 60.5) (width 0.2) (layer "F.Cu") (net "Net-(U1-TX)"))
 (segment (start 139 65) (end 143.5 60.5) (width 0.2) (layer "F.Cu") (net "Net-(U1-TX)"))
 (segment (start 139 71) (end 139 65) (width 0.2) (layer "F.Cu") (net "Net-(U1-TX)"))
 (segment (start 138.5 71.5) (end 139 71) (width 0.2) (layer "F.Cu") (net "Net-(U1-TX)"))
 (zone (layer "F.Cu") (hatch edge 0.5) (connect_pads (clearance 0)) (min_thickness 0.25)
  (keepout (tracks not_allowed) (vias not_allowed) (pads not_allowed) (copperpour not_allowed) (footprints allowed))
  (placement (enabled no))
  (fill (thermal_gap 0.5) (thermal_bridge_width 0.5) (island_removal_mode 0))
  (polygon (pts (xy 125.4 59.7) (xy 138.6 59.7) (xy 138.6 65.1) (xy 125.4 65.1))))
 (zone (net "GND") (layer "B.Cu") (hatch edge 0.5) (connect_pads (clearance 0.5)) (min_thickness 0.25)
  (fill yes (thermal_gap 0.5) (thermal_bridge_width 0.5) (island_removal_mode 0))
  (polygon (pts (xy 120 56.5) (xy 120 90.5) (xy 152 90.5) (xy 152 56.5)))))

